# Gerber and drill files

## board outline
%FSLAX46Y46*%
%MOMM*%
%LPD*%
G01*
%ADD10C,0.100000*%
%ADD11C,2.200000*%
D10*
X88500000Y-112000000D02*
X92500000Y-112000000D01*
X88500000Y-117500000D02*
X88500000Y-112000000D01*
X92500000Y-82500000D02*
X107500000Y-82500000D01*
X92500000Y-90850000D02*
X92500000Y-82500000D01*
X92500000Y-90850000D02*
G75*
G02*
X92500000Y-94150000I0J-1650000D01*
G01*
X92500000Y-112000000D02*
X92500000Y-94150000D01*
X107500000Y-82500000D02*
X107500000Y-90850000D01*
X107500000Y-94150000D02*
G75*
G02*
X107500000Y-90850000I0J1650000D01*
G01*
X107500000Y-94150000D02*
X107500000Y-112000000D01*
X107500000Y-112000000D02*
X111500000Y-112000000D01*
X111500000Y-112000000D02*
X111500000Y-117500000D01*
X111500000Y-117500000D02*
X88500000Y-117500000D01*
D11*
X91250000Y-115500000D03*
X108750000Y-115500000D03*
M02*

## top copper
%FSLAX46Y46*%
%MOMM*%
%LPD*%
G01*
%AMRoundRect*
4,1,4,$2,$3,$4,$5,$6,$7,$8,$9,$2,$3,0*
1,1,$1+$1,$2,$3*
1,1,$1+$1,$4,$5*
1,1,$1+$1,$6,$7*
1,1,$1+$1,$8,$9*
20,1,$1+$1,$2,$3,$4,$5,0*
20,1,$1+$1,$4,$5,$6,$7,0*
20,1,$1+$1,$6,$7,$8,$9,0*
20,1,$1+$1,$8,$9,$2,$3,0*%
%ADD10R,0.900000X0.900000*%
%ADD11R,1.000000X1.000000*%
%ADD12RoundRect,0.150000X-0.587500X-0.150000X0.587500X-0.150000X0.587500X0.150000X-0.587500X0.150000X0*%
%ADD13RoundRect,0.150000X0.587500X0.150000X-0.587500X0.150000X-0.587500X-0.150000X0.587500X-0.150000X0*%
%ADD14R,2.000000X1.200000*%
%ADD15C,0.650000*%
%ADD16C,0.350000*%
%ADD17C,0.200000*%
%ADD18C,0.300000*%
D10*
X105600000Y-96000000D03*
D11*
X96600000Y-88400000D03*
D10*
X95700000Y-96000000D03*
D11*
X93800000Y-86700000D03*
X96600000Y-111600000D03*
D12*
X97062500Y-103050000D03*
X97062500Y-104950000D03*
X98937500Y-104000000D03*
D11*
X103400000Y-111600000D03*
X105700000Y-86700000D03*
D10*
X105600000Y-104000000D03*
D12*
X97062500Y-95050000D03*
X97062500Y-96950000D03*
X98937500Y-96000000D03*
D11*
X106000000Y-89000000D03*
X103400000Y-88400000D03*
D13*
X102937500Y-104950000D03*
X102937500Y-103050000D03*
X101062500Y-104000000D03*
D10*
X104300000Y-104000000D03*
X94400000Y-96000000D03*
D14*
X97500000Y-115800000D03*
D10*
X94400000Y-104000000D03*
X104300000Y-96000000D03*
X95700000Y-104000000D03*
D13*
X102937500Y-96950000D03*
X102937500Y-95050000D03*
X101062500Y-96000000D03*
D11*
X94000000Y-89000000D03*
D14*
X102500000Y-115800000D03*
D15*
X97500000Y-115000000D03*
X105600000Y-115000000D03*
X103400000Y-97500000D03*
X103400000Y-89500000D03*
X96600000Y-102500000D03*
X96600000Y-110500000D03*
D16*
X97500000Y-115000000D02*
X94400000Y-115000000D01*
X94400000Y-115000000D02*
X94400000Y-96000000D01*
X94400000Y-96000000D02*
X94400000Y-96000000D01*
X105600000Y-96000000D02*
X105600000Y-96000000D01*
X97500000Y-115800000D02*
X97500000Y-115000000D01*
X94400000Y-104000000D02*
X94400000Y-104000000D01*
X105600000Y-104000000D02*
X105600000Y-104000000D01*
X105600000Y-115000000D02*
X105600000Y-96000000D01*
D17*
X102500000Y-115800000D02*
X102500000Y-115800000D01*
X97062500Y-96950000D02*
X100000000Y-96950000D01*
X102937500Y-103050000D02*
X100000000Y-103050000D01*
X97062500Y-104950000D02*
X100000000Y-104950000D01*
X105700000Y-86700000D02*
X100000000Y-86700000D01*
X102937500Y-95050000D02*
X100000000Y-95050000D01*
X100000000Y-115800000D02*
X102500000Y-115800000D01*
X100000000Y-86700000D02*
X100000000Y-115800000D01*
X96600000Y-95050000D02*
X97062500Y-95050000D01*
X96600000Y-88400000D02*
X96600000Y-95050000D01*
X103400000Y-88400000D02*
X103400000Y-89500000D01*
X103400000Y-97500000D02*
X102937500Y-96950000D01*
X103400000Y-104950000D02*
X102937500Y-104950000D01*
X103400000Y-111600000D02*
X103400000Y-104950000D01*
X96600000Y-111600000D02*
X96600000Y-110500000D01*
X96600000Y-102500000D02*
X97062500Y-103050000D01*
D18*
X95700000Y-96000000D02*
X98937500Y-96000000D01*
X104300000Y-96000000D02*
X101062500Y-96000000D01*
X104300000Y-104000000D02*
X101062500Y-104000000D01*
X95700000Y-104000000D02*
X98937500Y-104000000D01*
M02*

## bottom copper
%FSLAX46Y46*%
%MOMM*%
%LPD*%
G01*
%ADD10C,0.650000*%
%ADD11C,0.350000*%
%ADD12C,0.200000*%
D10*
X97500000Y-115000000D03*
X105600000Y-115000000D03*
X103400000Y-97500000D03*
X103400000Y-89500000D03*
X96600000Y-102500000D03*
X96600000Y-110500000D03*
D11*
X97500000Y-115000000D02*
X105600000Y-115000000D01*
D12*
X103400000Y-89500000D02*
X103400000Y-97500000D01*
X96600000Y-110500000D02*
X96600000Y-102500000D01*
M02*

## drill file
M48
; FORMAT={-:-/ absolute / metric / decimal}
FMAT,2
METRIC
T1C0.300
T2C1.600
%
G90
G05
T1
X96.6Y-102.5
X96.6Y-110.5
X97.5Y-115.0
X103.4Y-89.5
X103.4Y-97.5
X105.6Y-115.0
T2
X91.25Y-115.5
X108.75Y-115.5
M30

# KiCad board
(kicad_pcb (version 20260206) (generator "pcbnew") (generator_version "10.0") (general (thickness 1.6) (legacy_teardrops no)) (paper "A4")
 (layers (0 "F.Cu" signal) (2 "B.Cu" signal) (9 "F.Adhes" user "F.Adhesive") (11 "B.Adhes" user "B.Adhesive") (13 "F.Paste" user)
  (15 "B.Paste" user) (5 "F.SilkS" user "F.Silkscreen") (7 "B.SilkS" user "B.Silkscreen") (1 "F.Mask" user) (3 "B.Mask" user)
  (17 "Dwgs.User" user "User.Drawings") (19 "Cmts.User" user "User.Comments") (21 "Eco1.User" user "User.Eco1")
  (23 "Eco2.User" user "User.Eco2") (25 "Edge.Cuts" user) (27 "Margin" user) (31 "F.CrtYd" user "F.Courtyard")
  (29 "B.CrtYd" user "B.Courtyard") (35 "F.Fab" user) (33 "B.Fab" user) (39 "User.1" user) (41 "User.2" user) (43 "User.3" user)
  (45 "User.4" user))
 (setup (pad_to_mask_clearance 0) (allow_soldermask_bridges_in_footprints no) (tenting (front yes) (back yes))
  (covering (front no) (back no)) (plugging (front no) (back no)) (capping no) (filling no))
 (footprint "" (layer "F.Cu") (at 105.6 96)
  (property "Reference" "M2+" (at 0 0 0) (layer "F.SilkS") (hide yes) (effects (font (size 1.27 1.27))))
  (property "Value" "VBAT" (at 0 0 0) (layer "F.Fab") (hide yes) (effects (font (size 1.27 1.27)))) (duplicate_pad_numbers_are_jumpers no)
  (pad "1" smd rect (at 0 0) (size 0.9 0.9) (layers "F.Cu" "F.Mask" "F.Paste") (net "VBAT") (thermal_bridge_angle 45)))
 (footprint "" (layer "F.Cu") (at 96.6 88.4)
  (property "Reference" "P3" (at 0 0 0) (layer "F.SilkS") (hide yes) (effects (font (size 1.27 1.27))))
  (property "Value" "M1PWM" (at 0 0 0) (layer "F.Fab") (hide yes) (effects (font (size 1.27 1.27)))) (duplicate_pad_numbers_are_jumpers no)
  (pad "1" smd rect (at 0 0) (size 1 1) (layers "F.Cu" "F.Mask" "F.Paste") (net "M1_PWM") (thermal_bridge_angle 45)))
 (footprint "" (layer "F.Cu") (at 95.7 96)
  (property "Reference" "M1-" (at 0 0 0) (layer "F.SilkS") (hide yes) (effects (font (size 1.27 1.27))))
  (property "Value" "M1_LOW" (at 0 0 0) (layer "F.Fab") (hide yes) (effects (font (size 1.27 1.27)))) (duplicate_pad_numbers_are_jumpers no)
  (pad "1" smd rect (at 0 0) (size 0.9 0.9) (layers "F.Cu" "F.Mask" "F.Paste") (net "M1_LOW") (thermal_bridge_angle 45)))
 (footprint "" (layer "F.Cu") (at 93.8 86.7)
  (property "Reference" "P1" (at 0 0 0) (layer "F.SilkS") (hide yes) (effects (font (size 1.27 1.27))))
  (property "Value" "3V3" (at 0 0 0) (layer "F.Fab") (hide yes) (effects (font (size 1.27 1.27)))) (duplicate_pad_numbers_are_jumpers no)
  (pad "1" smd rect (at 0 0) (size 1 1) (layers "F.Cu" "F.Mask" "F.Paste") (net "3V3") (thermal_bridge_angle 45)))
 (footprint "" (layer "F.Cu") (at 96.6 111.6)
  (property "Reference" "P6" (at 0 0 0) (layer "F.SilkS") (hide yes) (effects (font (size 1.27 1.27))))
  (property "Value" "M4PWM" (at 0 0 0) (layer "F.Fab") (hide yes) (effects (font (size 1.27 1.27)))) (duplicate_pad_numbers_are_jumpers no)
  (pad "1" smd rect (at 0 0) (size 1 1) (layers "F.Cu" "F.Mask" "F.Paste") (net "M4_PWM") (thermal_bridge_angle 45)))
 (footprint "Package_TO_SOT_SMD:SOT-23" (layer "F.Cu") (at 98 104)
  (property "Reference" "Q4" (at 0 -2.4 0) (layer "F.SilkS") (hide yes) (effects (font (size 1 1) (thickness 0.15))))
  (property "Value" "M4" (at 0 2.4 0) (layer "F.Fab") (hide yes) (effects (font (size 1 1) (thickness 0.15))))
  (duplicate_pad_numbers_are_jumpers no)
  (pad "1" smd roundrect (at -0.9375 -0.95) (size 1.475 0.6) (layers "F.Cu" "F.Mask" "F.Paste") (roundrect_rratio 0.25) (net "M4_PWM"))
  (pad "2" smd roundrect (at -0.9375 0.95) (size 1.475 0.6) (layers "F.Cu" "F.Mask" "F.Paste") (roundrect_rratio 0.25) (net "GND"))
  (pad "3" smd roundrect (at 0.9375 0) (size 1.475 0.6) (layers "F.Cu" "F.Mask" "F.Paste") (roundrect_rratio 0.25) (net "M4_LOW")))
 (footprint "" (layer "F.Cu") (at 103.4 111.6)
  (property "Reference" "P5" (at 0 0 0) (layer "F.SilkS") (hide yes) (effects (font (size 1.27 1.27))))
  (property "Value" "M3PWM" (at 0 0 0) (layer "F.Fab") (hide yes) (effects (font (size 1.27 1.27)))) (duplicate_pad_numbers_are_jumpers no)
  (pad "1" smd rect (at 0 0) (size 1 1) (layers "F.Cu" "F.Mask" "F.Paste") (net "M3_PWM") (thermal_bridge_angle 45)))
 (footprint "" (layer "F.Cu") (at 105.7 86.7)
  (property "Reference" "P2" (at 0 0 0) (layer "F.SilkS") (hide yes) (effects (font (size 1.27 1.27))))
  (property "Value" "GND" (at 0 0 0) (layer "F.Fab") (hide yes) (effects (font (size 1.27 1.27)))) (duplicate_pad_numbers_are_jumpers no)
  (pad "1" smd rect (at 0 0) (size 1 1) (layers "F.Cu" "F.Mask" "F.Paste") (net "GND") (thermal_bridge_angle 45)))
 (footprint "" (layer "F.Cu") (at 105.6 104)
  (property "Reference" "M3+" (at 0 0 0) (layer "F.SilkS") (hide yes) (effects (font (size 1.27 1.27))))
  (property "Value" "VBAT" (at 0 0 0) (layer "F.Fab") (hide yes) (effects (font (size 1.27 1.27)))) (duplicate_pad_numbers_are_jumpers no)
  (pad "1" smd rect (at 0 0) (size 0.9 0.9) (layers "F.Cu" "F.Mask" "F.Paste") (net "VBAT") (thermal_bridge_angle 45)))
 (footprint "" (layer "F.Cu") (at 91.25 115.5)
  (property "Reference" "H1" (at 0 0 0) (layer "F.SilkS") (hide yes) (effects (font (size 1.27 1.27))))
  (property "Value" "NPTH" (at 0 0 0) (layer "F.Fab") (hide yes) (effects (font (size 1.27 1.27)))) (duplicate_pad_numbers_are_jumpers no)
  (pad "" np_thru_hole circle (at 0 0) (size 2.2 2.2) (drill 1.6) (layers "Edge.Cuts")))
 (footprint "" (layer "F.Cu") (at 108.75 115.5)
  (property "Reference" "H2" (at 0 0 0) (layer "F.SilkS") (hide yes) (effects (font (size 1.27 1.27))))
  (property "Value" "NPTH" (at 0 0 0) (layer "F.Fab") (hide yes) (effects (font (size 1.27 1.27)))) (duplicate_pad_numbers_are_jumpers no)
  (pad "" np_thru_hole circle (at 0 0) (size 2.2 2.2) (drill 1.6) (layers "Edge.Cuts")))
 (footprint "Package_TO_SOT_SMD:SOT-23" (layer "F.Cu") (at 98 96)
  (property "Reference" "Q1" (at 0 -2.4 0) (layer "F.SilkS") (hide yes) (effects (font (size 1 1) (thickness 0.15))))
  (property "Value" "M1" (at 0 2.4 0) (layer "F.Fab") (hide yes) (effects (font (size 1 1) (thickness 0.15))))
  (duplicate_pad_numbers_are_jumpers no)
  (pad "1" smd roundrect (at -0.9375 -0.95) (size 1.475 0.6) (layers "F.Cu" "F.Mask" "F.Paste") (roundrect_rratio 0.25) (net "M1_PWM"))
  (pad "2" smd roundrect (at -0.9375 0.95) (size 1.475 0.6) (layers "F.Cu" "F.Mask" "F.Paste") (roundrect_rratio 0.25) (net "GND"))
  (pad "3" smd roundrect (at 0.9375 0) (size 1.475 0.6) (layers "F.Cu" "F.Mask" "F.Paste") (roundrect_rratio 0.25) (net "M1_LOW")))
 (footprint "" (layer "F.Cu") (at 106 89)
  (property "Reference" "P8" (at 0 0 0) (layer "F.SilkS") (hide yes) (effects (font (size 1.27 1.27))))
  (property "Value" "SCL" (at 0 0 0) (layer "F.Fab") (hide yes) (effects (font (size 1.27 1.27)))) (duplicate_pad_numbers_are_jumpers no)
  (pad "1" smd rect (at 0 0) (size 1 1) (layers "F.Cu" "F.Mask" "F.Paste") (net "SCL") (thermal_bridge_angle 45)))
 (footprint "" (layer "F.Cu") (at 103.4 88.4)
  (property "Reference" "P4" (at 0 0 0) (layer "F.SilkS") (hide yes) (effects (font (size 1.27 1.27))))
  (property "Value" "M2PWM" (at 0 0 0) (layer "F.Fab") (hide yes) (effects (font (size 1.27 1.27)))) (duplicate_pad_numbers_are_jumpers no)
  (pad "1" smd rect (at 0 0) (size 1 1) (layers "F.Cu" "F.Mask" "F.Paste") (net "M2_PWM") (thermal_bridge_angle 45)))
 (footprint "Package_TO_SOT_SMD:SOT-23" (layer "F.Cu") (at 102 104 180)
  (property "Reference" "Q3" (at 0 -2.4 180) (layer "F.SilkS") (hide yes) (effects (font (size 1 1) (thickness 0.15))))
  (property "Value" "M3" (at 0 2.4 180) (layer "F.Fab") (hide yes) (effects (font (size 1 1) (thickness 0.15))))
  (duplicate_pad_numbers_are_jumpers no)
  (pad "1" smd roundrect (at -0.9375 -0.95 180) (size 1.475 0.6) (layers "F.Cu" "F.Mask" "F.Paste") (roundrect_rratio 0.25) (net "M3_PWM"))
  (pad "2" smd roundrect (at -0.9375 0.95 180) (size 1.475 0.6) (layers "F.Cu" "F.Mask" "F.Paste") (roundrect_rratio 0.25) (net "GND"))
  (pad "3" smd roundrect (at 0.9375 0 180) (size 1.475 0.6) (layers "F.Cu" "F.Mask" "F.Paste") (roundrect_rratio 0.25) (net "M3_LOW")))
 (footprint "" (layer "F.Cu") (at 104.3 104)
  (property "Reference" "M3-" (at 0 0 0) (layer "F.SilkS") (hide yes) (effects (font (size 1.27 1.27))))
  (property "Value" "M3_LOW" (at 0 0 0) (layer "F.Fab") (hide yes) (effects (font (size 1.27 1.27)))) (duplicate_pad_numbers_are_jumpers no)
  (pad "1" smd rect (at 0 0) (size 0.9 0.9) (layers "F.Cu" "F.Mask" "F.Paste") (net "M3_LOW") (thermal_bridge_angle 45)))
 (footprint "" (layer "F.Cu") (at 94.4 96)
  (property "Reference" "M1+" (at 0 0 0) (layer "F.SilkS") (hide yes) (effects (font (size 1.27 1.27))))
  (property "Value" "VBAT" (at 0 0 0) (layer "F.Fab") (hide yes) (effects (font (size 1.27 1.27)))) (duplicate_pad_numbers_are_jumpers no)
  (pad "1" smd rect (at 0 0) (size 0.9 0.9) (layers "F.Cu" "F.Mask" "F.Paste") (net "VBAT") (thermal_bridge_angle 45)))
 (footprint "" (layer "F.Cu") (at 97.5 115.8)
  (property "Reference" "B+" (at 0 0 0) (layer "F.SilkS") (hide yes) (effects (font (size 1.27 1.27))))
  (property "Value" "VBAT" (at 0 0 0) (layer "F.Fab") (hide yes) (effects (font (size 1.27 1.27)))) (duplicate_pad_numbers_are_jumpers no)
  (pad "1" smd rect (at 0 0) (size 2 1.2) (layers "F.Cu" "F.Mask" "F.Paste") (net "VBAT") (thermal_bridge_angle 45)))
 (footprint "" (layer "F.Cu") (at 94.4 104)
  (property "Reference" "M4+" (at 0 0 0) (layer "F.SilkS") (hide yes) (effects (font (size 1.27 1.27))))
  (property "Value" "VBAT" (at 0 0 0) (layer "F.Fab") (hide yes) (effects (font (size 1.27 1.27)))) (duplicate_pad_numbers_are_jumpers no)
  (pad "1" smd rect (at 0 0) (size 0.9 0.9) (layers "F.Cu" "F.Mask" "F.Paste") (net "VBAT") (thermal_bridge_angle 45)))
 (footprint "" (layer "F.Cu") (at 104.3 96)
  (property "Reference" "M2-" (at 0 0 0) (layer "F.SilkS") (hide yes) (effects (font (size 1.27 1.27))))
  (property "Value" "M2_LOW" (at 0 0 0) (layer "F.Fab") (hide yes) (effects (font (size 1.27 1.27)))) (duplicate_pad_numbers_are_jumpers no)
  (pad "1" smd rect (at 0 0) (size 0.9 0.9) (layers "F.Cu" "F.Mask" "F.Paste") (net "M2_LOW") (thermal_bridge_angle 45)))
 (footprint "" (layer "F.Cu") (at 95.7 104)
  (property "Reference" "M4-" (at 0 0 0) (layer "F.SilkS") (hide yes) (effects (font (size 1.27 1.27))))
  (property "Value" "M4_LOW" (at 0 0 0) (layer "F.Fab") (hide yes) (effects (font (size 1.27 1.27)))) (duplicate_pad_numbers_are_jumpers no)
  (pad "1" smd rect (at 0 0) (size 0.9 0.9) (layers "F.Cu" "F.Mask" "F.Paste") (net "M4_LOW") (thermal_bridge_angle 45)))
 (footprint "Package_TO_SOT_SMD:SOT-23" (layer "F.Cu") (at 102 96 180)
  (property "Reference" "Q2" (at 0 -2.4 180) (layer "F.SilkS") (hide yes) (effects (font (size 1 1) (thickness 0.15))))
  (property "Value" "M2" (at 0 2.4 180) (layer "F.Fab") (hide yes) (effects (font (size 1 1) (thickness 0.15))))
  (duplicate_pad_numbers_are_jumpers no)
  (pad "1" smd roundrect (at -0.9375 -0.95 180) (size 1.475 0.6) (layers "F.Cu" "F.Mask" "F.Paste") (roundrect_rratio 0.25) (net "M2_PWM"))
  (pad "2" smd roundrect (at -0.9375 0.95 180) (size 1.475 0.6) (layers "F.Cu" "F.Mask" "F.Paste") (roundrect_rratio 0.25) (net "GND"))
  (pad "3" smd roundrect (at 0.9375 0 180) (size 1.475 0.6) (layers "F.Cu" "F.Mask" "F.Paste") (roundrect_rratio 0.25) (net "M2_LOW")))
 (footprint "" (layer "F.Cu") (at 94 89)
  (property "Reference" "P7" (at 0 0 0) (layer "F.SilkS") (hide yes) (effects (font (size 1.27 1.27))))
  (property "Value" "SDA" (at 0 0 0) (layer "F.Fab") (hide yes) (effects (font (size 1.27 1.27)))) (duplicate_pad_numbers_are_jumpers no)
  (pad "1" smd rect (at 0 0) (size 1 1) (layers "F.Cu" "F.Mask" "F.Paste") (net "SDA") (thermal_bridge_angle 45)))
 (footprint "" (layer "F.Cu") (at 102.5 115.8)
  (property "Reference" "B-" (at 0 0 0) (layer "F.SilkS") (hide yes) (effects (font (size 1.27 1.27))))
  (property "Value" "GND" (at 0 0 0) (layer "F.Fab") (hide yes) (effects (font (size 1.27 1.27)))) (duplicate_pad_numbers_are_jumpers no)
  (pad "1" smd rect (at 0 0) (size 2 1.2) (layers "F.Cu" "F.Mask" "F.Paste") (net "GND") (thermal_bridge_angle 45)))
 (gr_line (start 88.5 112) (end 92.5 112) (stroke (width 0.1) (type default)) (layer "Edge.Cuts"))
 (gr_line (start 88.5 117.5) (end 88.5 112) (stroke (width 0.1) (type default)) (layer "Edge.Cuts"))
 (gr_line (start 92.5 82.5) (end 107.5 82.5) (stroke (width 0.1) (type default)) (layer "Edge.Cuts"))
 (gr_line (start 92.5 90.85) (end 92.5 82.5) (stroke (width 0.1) (type default)) (layer "Edge.Cuts"))
 (gr_arc (start 92.5 90.85) (mid 94.15 92.5) (end 92.5 94.15) (stroke (width 0.1) (type default)) (layer "Edge.Cuts"))
 (gr_line (start 92.5 112) (end 92.5 94.15) (stroke (width 0.1) (type default)) (layer "Edge.Cuts"))
 (gr_line (start 107.5 82.5) (end 107.5 90.85) (stroke (width 0.1) (type default)) (layer "Edge.Cuts"))
 (gr_arc (start 107.5 94.15) (mid 105.85 92.5) (end 107.5 90.85) (stroke (width 0.1) (type default)) (layer "Edge.Cuts"))
 (gr_line (start 107.5 94.15) (end 107.5 112) (stroke (width 0.1) (type default)) (layer "Edge.Cuts"))
 (gr_line (start 107.5 112) (end 111.5 112) (stroke (width 0.1) (type default)) (layer "Edge.Cuts"))
 (gr_line (start 111.5 112) (end 111.5 117.5) (stroke (width 0.1) (type default)) (layer "Edge.Cuts"))
 (gr_line (start 111.5 117.5) (end 88.5 117.5) (stroke (width 0.1) (type default)) (layer "Edge.Cuts"))
 (segment (start 97.5 115) (end 94.4 115) (width 0.35) (layer "F.Cu") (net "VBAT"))
 (segment (start 94.4 115) (end 94.4 96) (width 0.35) (layer "F.Cu") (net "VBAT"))
 (segment (start 94.4 96) (end 94.4 96) (width 0.35) (layer "F.Cu") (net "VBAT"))
 (segment (start 105.6 96) (end 105.6 96) (width 0.35) (layer "F.Cu") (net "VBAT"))
 (segment (start 97.5 115.8) (end 97.5 115) (width 0.35) (layer "F.Cu") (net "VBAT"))
 (segment (start 94.4 104) (end 94.4 104) (width 0.35) (layer "F.Cu") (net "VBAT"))
 (segment (start 105.6 104) (end 105.6 104) (width 0.35) (layer "F.Cu") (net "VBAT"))
 (segment (start 105.6 115) (end 105.6 96) (width 0.35) (layer "F.Cu") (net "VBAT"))
 (via (at 97.5 115) (size 0.65) (drill 0.3) (layers "F.Cu" "B.Cu") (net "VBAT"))
 (via (at 105.6 115) (size 0.65) (drill 0.3) (layers "F.Cu" "B.Cu") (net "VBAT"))
 (segment (start 97.5 115) (end 105.6 115) (width 0.35) (layer "B.Cu") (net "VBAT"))
 (segment (start 102.5 115.8) (end 102.5 115.8) (width 0.2) (layer "F.Cu") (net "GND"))
 (segment (start 97.0625 96.95) (end 100 96.95) (width 0.2) (layer "F.Cu") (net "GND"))
 (segment (start 102.9375 103.05) (end 100 103.05) (width 0.2) (layer "F.Cu") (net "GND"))
 (segment (start 97.0625 104.95) (end 100 104.95) (width 0.2) (layer "F.Cu") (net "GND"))
 (segment (start 105.7 86.7) (end 100 86.7) (width 0.2) (layer "F.Cu") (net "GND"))
 (segment (start 102.9375 95.05) (end 100 95.05) (width 0.2) (layer "F.Cu") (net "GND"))
 (segment (start 100 115.8) (end 102.5 115.8) (width 0.2) (layer "F.Cu") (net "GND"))
 (segment (start 100 86.7) (end 100 115.8) (width 0.2) (layer "F.Cu") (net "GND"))
 (segment (start 96.6 95.05) (end 97.0625 95.05) (width 0.2) (layer "F.Cu") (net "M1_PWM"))
 (segment (start 96.6 88.4) (end 96.6 95.05) (width 0.2) (layer "F.Cu") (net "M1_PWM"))
 (segment (start 103.4 88.4) (end 103.4 89.5) (width 0.2) (layer "F.Cu") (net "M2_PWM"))
 (segment (start 103.4 97.5) (end 102.9375 96.95) (width 0.2) (layer "F.Cu") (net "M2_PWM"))
 (via (at 103.4 97.5) (size 0.65) (drill 0.3) (layers "F.Cu" "B.Cu") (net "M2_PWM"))
 (via (at 103.4 89.5) (size 0.65) (drill 0.3) (layers "F.Cu" "B.Cu") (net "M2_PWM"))
 (segment (start 103.4 89.5) (end 103.4 97.5) (width 0.2) (layer "B.Cu") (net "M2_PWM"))
 (segment (start 103.4 104.95) (end 102.9375 104.95) (width 0.2) (layer "F.Cu") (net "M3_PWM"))
 (segment (start 103.4 111.6) (end 103.4 104.95) (width 0.2) (layer "F.Cu") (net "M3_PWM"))
 (segment (start 96.6 111.6) (end 96.6 110.5) (width 0.2) (layer "F.Cu") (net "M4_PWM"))
 (segment (start 96.6 102.5) (end 97.0625 103.05) (width 0.2) (layer "F.Cu") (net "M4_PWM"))
 (via (at 96.6 102.5) (size 0.65) (drill 0.3) (layers "F.Cu" "B.Cu") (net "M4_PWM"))
 (via (at 96.6 110.5) (size 0.65) (drill 0.3) (layers "F.Cu" "B.Cu") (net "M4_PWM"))
 (segment (start 96.6 110.5) (end 96.6 102.5) (width 0.2) (layer "B.Cu") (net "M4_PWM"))
 (segment (start 95.7 96) (end 98.9375 96) (width 0.3) (layer "F.Cu") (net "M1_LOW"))
 (segment (start 104.3 96) (end 101.0625 96) (width 0.3) (layer "F.Cu") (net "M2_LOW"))
 (segment (start 104.3 104) (end 101.0625 104) (width 0.3) (layer "F.Cu") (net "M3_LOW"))
 (segment (start 95.7 104) (end 98.9375 104) (width 0.3) (layer "F.Cu") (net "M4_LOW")))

